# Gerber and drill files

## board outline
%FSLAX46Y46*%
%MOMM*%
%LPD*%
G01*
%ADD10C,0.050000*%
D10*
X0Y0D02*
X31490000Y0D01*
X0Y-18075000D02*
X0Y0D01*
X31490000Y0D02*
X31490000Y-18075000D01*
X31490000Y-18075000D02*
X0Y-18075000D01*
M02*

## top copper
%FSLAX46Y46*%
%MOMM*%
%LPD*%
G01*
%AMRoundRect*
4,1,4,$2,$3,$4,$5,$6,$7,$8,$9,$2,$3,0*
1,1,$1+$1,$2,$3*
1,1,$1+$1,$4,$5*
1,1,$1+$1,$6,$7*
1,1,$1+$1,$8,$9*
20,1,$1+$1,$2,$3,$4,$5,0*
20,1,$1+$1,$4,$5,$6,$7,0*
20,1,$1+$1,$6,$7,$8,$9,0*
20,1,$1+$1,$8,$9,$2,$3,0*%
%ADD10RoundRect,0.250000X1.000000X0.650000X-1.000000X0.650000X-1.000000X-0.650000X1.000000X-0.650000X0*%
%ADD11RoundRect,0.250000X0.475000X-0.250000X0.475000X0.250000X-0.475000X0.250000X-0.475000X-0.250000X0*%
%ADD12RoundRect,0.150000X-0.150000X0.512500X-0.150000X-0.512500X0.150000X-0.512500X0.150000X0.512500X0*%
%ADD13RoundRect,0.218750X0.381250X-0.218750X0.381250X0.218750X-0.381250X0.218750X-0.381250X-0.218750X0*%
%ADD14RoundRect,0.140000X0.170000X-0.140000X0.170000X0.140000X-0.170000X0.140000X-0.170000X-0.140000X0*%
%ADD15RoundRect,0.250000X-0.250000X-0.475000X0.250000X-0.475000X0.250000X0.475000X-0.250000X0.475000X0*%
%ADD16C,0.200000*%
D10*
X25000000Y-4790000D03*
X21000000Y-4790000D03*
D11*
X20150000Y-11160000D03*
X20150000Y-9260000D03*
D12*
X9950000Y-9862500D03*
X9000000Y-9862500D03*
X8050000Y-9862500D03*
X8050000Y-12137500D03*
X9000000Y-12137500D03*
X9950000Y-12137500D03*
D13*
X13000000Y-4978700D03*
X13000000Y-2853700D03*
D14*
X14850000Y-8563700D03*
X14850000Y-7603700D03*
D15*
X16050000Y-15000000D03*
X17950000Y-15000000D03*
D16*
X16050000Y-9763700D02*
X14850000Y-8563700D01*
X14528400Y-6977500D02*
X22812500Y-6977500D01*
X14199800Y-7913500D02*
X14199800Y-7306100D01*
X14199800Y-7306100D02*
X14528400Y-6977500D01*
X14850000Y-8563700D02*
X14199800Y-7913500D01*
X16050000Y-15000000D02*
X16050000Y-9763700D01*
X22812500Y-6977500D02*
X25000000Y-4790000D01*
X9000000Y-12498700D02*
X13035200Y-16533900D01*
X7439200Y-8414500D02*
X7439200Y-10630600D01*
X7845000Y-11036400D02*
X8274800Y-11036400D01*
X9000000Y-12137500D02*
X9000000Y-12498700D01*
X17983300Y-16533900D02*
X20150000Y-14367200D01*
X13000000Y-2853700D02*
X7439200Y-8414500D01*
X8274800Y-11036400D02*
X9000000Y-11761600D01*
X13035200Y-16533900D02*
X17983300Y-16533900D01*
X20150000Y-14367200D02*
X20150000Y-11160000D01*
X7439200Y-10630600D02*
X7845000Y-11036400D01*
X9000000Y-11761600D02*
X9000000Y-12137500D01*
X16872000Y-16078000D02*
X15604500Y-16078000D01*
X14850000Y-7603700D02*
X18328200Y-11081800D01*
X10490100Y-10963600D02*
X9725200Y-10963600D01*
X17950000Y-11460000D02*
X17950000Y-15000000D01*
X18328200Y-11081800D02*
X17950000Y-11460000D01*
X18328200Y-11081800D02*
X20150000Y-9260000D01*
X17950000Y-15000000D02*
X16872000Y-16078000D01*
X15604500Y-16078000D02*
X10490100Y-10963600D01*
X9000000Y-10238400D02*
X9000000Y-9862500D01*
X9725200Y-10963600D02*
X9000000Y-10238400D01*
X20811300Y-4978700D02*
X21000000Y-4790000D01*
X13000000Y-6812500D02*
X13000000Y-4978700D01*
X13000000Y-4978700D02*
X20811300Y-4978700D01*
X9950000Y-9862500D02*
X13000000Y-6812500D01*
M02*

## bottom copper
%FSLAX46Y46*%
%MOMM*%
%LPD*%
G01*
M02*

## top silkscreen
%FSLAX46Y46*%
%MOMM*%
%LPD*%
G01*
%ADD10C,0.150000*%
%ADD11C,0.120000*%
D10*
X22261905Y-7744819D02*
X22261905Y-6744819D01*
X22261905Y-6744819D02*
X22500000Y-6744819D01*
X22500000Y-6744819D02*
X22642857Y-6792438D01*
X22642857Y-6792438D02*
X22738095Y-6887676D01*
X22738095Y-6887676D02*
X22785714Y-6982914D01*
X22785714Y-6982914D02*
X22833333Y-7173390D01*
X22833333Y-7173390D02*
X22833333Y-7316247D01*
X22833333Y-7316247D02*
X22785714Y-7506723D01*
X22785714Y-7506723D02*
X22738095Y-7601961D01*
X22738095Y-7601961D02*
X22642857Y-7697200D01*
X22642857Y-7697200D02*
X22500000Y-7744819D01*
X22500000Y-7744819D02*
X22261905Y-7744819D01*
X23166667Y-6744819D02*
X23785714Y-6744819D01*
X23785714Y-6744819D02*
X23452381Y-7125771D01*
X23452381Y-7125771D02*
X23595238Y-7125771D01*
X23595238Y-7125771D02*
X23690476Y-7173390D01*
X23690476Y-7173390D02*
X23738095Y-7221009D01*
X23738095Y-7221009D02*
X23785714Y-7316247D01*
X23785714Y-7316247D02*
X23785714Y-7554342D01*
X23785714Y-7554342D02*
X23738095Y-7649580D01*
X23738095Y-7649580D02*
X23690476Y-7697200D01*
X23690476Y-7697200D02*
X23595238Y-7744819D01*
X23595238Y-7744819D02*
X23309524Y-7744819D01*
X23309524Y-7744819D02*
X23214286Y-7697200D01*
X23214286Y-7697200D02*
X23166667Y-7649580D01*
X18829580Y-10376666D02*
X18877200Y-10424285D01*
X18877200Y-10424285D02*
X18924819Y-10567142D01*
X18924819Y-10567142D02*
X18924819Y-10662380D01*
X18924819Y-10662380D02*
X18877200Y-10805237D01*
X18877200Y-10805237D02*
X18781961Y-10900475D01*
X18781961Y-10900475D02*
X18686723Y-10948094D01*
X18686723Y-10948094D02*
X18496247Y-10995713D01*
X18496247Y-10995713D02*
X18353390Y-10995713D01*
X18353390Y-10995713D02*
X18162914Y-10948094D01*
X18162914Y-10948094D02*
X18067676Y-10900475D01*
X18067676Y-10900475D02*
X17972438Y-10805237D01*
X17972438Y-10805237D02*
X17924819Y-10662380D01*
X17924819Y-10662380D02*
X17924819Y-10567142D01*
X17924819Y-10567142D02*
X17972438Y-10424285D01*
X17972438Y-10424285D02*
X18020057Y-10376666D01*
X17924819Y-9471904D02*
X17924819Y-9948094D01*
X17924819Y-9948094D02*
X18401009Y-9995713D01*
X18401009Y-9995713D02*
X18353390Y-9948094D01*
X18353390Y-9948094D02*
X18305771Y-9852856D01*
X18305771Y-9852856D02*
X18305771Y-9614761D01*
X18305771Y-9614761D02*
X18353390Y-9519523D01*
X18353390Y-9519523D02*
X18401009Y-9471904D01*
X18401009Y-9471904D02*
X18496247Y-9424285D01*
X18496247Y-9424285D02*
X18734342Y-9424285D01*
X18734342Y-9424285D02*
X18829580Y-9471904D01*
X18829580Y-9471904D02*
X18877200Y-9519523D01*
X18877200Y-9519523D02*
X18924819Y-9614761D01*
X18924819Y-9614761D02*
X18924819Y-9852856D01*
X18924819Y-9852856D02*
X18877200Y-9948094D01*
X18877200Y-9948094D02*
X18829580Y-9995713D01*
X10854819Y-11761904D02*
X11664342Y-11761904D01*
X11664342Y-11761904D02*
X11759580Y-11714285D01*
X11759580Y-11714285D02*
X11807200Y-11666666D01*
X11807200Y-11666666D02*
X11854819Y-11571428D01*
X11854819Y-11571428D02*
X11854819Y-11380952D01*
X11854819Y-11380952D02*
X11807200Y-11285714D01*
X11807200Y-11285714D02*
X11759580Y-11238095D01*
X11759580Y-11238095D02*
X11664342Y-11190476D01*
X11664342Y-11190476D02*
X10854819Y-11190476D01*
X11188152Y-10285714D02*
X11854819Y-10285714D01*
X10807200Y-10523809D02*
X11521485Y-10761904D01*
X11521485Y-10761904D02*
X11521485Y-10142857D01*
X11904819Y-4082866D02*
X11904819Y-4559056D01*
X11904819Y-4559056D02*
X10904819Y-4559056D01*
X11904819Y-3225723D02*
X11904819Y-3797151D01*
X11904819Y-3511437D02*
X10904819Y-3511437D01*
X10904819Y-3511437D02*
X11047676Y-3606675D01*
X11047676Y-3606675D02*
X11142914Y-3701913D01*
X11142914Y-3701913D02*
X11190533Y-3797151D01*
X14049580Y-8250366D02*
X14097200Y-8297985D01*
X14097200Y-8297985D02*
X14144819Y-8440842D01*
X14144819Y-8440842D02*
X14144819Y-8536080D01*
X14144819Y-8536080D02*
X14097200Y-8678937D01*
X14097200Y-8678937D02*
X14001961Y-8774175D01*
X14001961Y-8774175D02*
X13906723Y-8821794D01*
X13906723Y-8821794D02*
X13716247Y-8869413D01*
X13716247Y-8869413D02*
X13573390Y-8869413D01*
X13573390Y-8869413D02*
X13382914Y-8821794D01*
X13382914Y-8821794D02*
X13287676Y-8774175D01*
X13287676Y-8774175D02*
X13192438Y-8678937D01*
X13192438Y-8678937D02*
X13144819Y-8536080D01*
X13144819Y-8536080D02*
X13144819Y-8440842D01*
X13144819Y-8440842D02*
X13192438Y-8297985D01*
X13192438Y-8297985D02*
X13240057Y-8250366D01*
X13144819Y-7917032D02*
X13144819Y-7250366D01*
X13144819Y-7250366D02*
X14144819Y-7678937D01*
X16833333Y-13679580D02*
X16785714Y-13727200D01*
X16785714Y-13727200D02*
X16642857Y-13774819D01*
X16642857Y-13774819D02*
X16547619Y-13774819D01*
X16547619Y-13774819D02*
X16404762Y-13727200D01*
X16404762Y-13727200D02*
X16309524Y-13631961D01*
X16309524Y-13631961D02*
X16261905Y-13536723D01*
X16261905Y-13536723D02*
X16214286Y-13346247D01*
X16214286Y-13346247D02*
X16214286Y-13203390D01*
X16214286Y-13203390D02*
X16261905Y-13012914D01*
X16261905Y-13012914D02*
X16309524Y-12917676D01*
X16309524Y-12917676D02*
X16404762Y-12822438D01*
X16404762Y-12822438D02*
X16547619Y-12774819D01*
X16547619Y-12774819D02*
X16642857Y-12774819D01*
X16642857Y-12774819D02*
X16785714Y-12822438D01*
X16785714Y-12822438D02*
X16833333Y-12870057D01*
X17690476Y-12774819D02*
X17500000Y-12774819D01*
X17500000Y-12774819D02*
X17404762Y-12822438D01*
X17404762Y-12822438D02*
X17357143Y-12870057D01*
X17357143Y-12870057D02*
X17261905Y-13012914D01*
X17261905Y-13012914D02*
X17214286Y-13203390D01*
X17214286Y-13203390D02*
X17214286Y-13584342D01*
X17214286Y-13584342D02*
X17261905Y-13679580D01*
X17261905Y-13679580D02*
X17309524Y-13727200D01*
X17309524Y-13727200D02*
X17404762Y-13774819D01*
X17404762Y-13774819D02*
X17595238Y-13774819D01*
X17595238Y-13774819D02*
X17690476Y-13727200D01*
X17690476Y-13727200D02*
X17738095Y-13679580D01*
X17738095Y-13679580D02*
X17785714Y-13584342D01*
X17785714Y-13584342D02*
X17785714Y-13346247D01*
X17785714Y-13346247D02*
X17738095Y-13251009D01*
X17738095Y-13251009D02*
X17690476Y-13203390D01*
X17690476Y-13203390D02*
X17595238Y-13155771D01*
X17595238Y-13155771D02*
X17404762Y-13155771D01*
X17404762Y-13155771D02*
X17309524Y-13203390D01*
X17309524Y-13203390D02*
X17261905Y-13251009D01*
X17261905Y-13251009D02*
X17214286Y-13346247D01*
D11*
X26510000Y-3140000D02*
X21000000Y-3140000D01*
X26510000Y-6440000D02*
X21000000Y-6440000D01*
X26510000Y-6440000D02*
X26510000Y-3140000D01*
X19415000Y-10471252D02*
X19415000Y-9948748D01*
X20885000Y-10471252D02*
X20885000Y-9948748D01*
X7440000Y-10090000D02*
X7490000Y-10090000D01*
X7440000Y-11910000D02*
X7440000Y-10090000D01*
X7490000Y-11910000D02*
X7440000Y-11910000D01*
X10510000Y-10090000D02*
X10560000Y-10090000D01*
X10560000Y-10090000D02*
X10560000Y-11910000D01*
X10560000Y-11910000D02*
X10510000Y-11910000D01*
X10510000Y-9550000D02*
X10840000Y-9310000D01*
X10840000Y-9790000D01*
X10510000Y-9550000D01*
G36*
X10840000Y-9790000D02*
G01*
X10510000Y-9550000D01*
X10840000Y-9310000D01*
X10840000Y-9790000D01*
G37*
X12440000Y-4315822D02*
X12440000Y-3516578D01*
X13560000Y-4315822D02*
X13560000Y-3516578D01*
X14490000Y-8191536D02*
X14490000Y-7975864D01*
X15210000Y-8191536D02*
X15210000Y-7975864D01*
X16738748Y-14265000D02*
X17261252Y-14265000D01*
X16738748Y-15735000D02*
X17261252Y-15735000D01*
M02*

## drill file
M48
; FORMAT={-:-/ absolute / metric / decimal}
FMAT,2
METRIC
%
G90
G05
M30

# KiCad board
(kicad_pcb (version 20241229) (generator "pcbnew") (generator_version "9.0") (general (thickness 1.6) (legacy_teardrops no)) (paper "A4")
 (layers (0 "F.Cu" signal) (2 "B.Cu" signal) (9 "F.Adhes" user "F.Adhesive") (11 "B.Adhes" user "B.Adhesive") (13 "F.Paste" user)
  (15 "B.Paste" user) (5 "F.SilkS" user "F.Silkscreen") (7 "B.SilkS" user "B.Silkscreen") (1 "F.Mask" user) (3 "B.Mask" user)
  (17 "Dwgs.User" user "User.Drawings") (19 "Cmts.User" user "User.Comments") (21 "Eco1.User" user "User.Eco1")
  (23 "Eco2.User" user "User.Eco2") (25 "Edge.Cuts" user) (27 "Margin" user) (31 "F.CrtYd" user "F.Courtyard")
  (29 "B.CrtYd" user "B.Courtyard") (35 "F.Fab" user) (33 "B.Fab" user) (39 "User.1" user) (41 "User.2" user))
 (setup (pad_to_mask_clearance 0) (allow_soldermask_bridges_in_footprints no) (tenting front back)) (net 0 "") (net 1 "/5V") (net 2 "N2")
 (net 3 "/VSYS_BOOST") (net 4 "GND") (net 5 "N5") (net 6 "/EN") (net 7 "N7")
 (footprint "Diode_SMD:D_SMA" (layer "F.Cu") (at 23 4.79 180)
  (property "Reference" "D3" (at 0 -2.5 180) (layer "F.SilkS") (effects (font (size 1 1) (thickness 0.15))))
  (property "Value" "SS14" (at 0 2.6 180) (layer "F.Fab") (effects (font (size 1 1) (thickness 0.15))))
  (fp_line (start -3.51 1.65) (end 2 1.65) (stroke (width 0.12) (type solid)) (layer "F.SilkS"))
  (fp_line (start -3.51 -1.65) (end 2 -1.65) (stroke (width 0.12) (type solid)) (layer "F.SilkS"))
  (fp_line (start -3.51 -1.65) (end -3.51 1.65) (stroke (width 0.12) (type solid)) (layer "F.SilkS"))
  (pad "1" smd roundrect (at -2 0 180) (size 2.5 1.8) (layers "F.Cu" "F.Mask" "F.Paste") (roundrect_rratio 0.1388888889) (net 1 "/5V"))
  (pad "2" smd roundrect (at 2 0 180) (size 2.5 1.8) (layers "F.Cu" "F.Mask" "F.Paste") (roundrect_rratio 0.1388888889) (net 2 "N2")))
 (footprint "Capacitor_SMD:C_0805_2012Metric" (layer "F.Cu") (at 20.15 10.21 90)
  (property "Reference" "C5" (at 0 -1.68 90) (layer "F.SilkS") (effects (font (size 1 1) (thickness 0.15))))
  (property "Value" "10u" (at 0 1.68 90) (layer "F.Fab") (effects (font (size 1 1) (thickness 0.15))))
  (fp_line (start -0.261252 -0.735) (end 0.261252 -0.735) (stroke (width 0.12) (type solid)) (layer "F.SilkS"))
  (fp_line (start -0.261252 0.735) (end 0.261252 0.735) (stroke (width 0.12) (type solid)) (layer "F.SilkS"))
  (pad "1" smd roundrect (at -0.95 0 90) (size 1 1.45) (layers "F.Cu" "F.Mask" "F.Paste") (roundrect_rratio 0.25) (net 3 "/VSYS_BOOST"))
  (pad "2" smd roundrect (at 0.95 0 90) (size 1 1.45) (layers "F.Cu" "F.Mask" "F.Paste") (roundrect_rratio 0.25) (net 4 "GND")))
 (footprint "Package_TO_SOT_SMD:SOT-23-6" (layer "F.Cu") (at 9 11 -90)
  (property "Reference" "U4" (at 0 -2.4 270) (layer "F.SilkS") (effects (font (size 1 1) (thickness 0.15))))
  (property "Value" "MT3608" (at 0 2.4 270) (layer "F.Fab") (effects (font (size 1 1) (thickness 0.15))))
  (fp_line (start -0.91 1.56) (end -0.91 1.51) (stroke (width 0.12) (type solid)) (layer "F.SilkS"))
  (fp_line (start 0.91 1.56) (end -0.91 1.56) (stroke (width 0.12) (type solid)) (layer "F.SilkS"))
  (fp_line (start 0.91 1.51) (end 0.91 1.56) (stroke (width 0.12) (type solid)) (layer "F.SilkS"))
  (fp_line (start -0.91 -1.51) (end -0.91 -1.56) (stroke (width 0.12) (type solid)) (layer "F.SilkS"))
  (fp_line (start -0.91 -1.56) (end 0.91 -1.56) (stroke (width 0.12) (type solid)) (layer "F.SilkS"))
  (fp_line (start 0.91 -1.56) (end 0.91 -1.51) (stroke (width 0.12) (type solid)) (layer "F.SilkS"))
  (fp_poly (pts (xy -1.45 -1.51) (xy -1.69 -1.84) (xy -1.21 -1.84)) (stroke (width 0.12) (type solid)) (fill yes) (layer "F.SilkS"))
  (pad "1" smd roundrect (at -1.1375 -0.95 270) (size 1.325 0.6) (layers "F.Cu" "F.Mask" "F.Paste") (roundrect_rratio 0.25) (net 2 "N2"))
  (pad "2" smd roundrect (at -1.1375 0 270) (size 1.325 0.6) (layers "F.Cu" "F.Mask" "F.Paste") (roundrect_rratio 0.25) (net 4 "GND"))
  (pad "3" smd roundrect (at -1.1375 0.95 270) (size 1.325 0.6) (layers "F.Cu" "F.Mask" "F.Paste") (roundrect_rratio 0.25) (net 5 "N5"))
  (pad "4" smd roundrect (at 1.1375 0.95 270) (size 1.325 0.6) (layers "F.Cu" "F.Mask" "F.Paste") (roundrect_rratio 0.25) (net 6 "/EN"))
  (pad "5" smd roundrect (at 1.1375 0 270) (size 1.325 0.6) (layers "F.Cu" "F.Mask" "F.Paste") (roundrect_rratio 0.25) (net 3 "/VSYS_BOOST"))
  (pad "6" smd roundrect (at 1.1375 -0.95 270) (size 1.325 0.6) (layers "F.Cu" "F.Mask" "F.Paste") (roundrect_rratio 0.25) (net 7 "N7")))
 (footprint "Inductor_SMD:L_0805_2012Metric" (layer "F.Cu") (at 13 3.9162 90)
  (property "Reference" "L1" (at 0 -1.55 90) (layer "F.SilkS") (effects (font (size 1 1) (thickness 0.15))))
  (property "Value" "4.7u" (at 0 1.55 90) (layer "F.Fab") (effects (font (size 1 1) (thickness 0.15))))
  (fp_line (start -0.399622 -0.56) (end 0.399622 -0.56) (stroke (width 0.12) (type solid)) (layer "F.SilkS"))
  (fp_line (start -0.399622 0.56) (end 0.399622 0.56) (stroke (width 0.12) (type solid)) (layer "F.SilkS"))
  (pad "1" smd roundrect (at -1.0625 0 90) (size 0.875 1.2) (layers "F.Cu" "F.Mask" "F.Paste") (roundrect_rratio 0.25) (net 2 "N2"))
  (pad "2" smd roundrect (at 1.0625 0 90) (size 0.875 1.2) (layers "F.Cu" "F.Mask" "F.Paste") (roundrect_rratio 0.25) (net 3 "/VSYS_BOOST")))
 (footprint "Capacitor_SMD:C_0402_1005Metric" (layer "F.Cu") (at 14.85 8.0837 90)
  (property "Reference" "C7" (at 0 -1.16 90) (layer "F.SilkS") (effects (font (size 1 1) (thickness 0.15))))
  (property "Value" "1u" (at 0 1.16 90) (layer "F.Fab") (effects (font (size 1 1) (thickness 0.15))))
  (fp_line (start -0.107836 -0.36) (end 0.107836 -0.36) (stroke (width 0.12) (type solid)) (layer "F.SilkS"))
  (fp_line (start -0.107836 0.36) (end 0.107836 0.36) (stroke (width 0.12) (type solid)) (layer "F.SilkS"))
  (pad "1" smd roundrect (at -0.48 0 90) (size 0.56 0.62) (layers "F.Cu" "F.Mask" "F.Paste") (roundrect_rratio 0.25) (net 1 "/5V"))
  (pad "2" smd roundrect (at 0.48 0 90) (size 0.56 0.62) (layers "F.Cu" "F.Mask" "F.Paste") (roundrect_rratio 0.25) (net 4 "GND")))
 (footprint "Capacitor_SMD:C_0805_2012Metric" (layer "F.Cu") (at 17 15)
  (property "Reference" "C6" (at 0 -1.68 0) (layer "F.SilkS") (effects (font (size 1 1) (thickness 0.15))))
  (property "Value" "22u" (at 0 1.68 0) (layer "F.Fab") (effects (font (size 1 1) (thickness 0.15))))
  (fp_line (start -0.261252 -0.735) (end 0.261252 -0.735) (stroke (width 0.12) (type solid)) (layer "F.SilkS"))
  (fp_line (start -0.261252 0.735) (end 0.261252 0.735) (stroke (width 0.12) (type solid)) (layer "F.SilkS"))
  (pad "1" smd roundrect (at -0.95 0) (size 1 1.45) (layers "F.Cu" "F.Mask" "F.Paste") (roundrect_rratio 0.25) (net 1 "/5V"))
  (pad "2" smd roundrect (at 0.95 0) (size 1 1.45) (layers "F.Cu" "F.Mask" "F.Paste") (roundrect_rratio 0.25) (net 4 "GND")))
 (gr_line (start 0 0) (end 31.49 0) (stroke (width 0.05) (type default)) (layer "Edge.Cuts"))
 (gr_line (start 0 18.075) (end 0 0) (stroke (width 0.05) (type default)) (layer "Edge.Cuts"))
 (gr_line (start 31.49 0) (end 31.49 18.075) (stroke (width 0.05) (type default)) (layer "Edge.Cuts"))
 (gr_line (start 31.49 18.075) (end 0 18.075) (stroke (width 0.05) (type default)) (layer "Edge.Cuts"))
 (segment (start 16.05 9.7637) (end 14.85 8.5637) (width 0.2) (layer "F.Cu") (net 1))
 (segment (start 14.5284 6.9775) (end 22.8125 6.9775) (width 0.2) (layer "F.Cu") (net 1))
 (segment (start 14.1998 7.9135) (end 14.1998 7.3061) (width 0.2) (layer "F.Cu") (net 1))
 (segment (start 14.1998 7.3061) (end 14.5284 6.9775) (width 0.2) (layer "F.Cu") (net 1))
 (segment (start 14.85 8.5637) (end 14.1998 7.9135) (width 0.2) (layer "F.Cu") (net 1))
 (segment (start 16.05 15) (end 16.05 9.7637) (width 0.2) (layer "F.Cu") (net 1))
 (segment (start 22.8125 6.9775) (end 25 4.79) (width 0.2) (layer "F.Cu") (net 1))
 (segment (start 9 12.4987) (end 13.0352 16.5339) (width 0.2) (layer "F.Cu") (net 3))
 (segment (start 7.4392 8.4145) (end 7.4392 10.6306) (width 0.2) (layer "F.Cu") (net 3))
 (segment (start 7.845 11.0364) (end 8.2748 11.0364) (width 0.2) (layer "F.Cu") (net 3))
 (segment (start 9 12.1375) (end 9 12.4987) (width 0.2) (layer "F.Cu") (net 3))
 (segment (start 17.9833 16.5339) (end 20.15 14.3672) (width 0.2) (layer "F.Cu") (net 3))
 (segment (start 13 2.8537) (end 7.4392 8.4145) (width 0.2) (layer "F.Cu") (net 3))
 (segment (start 8.2748 11.0364) (end 9 11.7616) (width 0.2) (layer "F.Cu") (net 3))
 (segment (start 13.0352 16.5339) (end 17.9833 16.5339) (width 0.2) (layer "F.Cu") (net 3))
 (segment (start 20.15 14.3672) (end 20.15 11.16) (width 0.2) (layer "F.Cu") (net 3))
 (segment (start 7.4392 10.6306) (end 7.845 11.0364) (width 0.2) (layer "F.Cu") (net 3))
 (segment (start 9 11.7616) (end 9 12.1375) (width 0.2) (layer "F.Cu") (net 3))
 (segment (start 16.872 16.078) (end 15.6045 16.078) (width 0.2) (layer "F.Cu") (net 4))
 (segment (start 14.85 7.6037) (end 18.3282 11.0818) (width 0.2) (layer "F.Cu") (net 4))
 (segment (start 10.4901 10.9636) (end 9.7252 10.9636) (width 0.2) (layer "F.Cu") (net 4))
 (segment (start 17.95 11.46) (end 17.95 15) (width 0.2) (layer "F.Cu") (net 4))
 (segment (start 18.3282 11.0818) (end 17.95 11.46) (width 0.2) (layer "F.Cu") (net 4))
 (segment (start 18.3282 11.0818) (end 20.15 9.26) (width 0.2) (layer "F.Cu") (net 4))
 (segment (start 17.95 15) (end 16.872 16.078) (width 0.2) (layer "F.Cu") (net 4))
 (segment (start 15.6045 16.078) (end 10.4901 10.9636) (width 0.2) (layer "F.Cu") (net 4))
 (segment (start 9 10.2384) (end 9 9.8625) (width 0.2) (layer "F.Cu") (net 4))
 (segment (start 9.7252 10.9636) (end 9 10.2384) (width 0.2) (layer "F.Cu") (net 4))
 (segment (start 20.8113 4.9787) (end 21 4.79) (width 0.2) (layer "F.Cu") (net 2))
 (segment (start 13 6.8125) (end 13 4.9787) (width 0.2) (layer "F.Cu") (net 2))
 (segment (start 13 4.9787) (end 20.8113 4.9787) (width 0.2) (layer "F.Cu") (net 2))
 (segment (start 9.95 9.8625) (end 13 6.8125) (width 0.2) (layer "F.Cu") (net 2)))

